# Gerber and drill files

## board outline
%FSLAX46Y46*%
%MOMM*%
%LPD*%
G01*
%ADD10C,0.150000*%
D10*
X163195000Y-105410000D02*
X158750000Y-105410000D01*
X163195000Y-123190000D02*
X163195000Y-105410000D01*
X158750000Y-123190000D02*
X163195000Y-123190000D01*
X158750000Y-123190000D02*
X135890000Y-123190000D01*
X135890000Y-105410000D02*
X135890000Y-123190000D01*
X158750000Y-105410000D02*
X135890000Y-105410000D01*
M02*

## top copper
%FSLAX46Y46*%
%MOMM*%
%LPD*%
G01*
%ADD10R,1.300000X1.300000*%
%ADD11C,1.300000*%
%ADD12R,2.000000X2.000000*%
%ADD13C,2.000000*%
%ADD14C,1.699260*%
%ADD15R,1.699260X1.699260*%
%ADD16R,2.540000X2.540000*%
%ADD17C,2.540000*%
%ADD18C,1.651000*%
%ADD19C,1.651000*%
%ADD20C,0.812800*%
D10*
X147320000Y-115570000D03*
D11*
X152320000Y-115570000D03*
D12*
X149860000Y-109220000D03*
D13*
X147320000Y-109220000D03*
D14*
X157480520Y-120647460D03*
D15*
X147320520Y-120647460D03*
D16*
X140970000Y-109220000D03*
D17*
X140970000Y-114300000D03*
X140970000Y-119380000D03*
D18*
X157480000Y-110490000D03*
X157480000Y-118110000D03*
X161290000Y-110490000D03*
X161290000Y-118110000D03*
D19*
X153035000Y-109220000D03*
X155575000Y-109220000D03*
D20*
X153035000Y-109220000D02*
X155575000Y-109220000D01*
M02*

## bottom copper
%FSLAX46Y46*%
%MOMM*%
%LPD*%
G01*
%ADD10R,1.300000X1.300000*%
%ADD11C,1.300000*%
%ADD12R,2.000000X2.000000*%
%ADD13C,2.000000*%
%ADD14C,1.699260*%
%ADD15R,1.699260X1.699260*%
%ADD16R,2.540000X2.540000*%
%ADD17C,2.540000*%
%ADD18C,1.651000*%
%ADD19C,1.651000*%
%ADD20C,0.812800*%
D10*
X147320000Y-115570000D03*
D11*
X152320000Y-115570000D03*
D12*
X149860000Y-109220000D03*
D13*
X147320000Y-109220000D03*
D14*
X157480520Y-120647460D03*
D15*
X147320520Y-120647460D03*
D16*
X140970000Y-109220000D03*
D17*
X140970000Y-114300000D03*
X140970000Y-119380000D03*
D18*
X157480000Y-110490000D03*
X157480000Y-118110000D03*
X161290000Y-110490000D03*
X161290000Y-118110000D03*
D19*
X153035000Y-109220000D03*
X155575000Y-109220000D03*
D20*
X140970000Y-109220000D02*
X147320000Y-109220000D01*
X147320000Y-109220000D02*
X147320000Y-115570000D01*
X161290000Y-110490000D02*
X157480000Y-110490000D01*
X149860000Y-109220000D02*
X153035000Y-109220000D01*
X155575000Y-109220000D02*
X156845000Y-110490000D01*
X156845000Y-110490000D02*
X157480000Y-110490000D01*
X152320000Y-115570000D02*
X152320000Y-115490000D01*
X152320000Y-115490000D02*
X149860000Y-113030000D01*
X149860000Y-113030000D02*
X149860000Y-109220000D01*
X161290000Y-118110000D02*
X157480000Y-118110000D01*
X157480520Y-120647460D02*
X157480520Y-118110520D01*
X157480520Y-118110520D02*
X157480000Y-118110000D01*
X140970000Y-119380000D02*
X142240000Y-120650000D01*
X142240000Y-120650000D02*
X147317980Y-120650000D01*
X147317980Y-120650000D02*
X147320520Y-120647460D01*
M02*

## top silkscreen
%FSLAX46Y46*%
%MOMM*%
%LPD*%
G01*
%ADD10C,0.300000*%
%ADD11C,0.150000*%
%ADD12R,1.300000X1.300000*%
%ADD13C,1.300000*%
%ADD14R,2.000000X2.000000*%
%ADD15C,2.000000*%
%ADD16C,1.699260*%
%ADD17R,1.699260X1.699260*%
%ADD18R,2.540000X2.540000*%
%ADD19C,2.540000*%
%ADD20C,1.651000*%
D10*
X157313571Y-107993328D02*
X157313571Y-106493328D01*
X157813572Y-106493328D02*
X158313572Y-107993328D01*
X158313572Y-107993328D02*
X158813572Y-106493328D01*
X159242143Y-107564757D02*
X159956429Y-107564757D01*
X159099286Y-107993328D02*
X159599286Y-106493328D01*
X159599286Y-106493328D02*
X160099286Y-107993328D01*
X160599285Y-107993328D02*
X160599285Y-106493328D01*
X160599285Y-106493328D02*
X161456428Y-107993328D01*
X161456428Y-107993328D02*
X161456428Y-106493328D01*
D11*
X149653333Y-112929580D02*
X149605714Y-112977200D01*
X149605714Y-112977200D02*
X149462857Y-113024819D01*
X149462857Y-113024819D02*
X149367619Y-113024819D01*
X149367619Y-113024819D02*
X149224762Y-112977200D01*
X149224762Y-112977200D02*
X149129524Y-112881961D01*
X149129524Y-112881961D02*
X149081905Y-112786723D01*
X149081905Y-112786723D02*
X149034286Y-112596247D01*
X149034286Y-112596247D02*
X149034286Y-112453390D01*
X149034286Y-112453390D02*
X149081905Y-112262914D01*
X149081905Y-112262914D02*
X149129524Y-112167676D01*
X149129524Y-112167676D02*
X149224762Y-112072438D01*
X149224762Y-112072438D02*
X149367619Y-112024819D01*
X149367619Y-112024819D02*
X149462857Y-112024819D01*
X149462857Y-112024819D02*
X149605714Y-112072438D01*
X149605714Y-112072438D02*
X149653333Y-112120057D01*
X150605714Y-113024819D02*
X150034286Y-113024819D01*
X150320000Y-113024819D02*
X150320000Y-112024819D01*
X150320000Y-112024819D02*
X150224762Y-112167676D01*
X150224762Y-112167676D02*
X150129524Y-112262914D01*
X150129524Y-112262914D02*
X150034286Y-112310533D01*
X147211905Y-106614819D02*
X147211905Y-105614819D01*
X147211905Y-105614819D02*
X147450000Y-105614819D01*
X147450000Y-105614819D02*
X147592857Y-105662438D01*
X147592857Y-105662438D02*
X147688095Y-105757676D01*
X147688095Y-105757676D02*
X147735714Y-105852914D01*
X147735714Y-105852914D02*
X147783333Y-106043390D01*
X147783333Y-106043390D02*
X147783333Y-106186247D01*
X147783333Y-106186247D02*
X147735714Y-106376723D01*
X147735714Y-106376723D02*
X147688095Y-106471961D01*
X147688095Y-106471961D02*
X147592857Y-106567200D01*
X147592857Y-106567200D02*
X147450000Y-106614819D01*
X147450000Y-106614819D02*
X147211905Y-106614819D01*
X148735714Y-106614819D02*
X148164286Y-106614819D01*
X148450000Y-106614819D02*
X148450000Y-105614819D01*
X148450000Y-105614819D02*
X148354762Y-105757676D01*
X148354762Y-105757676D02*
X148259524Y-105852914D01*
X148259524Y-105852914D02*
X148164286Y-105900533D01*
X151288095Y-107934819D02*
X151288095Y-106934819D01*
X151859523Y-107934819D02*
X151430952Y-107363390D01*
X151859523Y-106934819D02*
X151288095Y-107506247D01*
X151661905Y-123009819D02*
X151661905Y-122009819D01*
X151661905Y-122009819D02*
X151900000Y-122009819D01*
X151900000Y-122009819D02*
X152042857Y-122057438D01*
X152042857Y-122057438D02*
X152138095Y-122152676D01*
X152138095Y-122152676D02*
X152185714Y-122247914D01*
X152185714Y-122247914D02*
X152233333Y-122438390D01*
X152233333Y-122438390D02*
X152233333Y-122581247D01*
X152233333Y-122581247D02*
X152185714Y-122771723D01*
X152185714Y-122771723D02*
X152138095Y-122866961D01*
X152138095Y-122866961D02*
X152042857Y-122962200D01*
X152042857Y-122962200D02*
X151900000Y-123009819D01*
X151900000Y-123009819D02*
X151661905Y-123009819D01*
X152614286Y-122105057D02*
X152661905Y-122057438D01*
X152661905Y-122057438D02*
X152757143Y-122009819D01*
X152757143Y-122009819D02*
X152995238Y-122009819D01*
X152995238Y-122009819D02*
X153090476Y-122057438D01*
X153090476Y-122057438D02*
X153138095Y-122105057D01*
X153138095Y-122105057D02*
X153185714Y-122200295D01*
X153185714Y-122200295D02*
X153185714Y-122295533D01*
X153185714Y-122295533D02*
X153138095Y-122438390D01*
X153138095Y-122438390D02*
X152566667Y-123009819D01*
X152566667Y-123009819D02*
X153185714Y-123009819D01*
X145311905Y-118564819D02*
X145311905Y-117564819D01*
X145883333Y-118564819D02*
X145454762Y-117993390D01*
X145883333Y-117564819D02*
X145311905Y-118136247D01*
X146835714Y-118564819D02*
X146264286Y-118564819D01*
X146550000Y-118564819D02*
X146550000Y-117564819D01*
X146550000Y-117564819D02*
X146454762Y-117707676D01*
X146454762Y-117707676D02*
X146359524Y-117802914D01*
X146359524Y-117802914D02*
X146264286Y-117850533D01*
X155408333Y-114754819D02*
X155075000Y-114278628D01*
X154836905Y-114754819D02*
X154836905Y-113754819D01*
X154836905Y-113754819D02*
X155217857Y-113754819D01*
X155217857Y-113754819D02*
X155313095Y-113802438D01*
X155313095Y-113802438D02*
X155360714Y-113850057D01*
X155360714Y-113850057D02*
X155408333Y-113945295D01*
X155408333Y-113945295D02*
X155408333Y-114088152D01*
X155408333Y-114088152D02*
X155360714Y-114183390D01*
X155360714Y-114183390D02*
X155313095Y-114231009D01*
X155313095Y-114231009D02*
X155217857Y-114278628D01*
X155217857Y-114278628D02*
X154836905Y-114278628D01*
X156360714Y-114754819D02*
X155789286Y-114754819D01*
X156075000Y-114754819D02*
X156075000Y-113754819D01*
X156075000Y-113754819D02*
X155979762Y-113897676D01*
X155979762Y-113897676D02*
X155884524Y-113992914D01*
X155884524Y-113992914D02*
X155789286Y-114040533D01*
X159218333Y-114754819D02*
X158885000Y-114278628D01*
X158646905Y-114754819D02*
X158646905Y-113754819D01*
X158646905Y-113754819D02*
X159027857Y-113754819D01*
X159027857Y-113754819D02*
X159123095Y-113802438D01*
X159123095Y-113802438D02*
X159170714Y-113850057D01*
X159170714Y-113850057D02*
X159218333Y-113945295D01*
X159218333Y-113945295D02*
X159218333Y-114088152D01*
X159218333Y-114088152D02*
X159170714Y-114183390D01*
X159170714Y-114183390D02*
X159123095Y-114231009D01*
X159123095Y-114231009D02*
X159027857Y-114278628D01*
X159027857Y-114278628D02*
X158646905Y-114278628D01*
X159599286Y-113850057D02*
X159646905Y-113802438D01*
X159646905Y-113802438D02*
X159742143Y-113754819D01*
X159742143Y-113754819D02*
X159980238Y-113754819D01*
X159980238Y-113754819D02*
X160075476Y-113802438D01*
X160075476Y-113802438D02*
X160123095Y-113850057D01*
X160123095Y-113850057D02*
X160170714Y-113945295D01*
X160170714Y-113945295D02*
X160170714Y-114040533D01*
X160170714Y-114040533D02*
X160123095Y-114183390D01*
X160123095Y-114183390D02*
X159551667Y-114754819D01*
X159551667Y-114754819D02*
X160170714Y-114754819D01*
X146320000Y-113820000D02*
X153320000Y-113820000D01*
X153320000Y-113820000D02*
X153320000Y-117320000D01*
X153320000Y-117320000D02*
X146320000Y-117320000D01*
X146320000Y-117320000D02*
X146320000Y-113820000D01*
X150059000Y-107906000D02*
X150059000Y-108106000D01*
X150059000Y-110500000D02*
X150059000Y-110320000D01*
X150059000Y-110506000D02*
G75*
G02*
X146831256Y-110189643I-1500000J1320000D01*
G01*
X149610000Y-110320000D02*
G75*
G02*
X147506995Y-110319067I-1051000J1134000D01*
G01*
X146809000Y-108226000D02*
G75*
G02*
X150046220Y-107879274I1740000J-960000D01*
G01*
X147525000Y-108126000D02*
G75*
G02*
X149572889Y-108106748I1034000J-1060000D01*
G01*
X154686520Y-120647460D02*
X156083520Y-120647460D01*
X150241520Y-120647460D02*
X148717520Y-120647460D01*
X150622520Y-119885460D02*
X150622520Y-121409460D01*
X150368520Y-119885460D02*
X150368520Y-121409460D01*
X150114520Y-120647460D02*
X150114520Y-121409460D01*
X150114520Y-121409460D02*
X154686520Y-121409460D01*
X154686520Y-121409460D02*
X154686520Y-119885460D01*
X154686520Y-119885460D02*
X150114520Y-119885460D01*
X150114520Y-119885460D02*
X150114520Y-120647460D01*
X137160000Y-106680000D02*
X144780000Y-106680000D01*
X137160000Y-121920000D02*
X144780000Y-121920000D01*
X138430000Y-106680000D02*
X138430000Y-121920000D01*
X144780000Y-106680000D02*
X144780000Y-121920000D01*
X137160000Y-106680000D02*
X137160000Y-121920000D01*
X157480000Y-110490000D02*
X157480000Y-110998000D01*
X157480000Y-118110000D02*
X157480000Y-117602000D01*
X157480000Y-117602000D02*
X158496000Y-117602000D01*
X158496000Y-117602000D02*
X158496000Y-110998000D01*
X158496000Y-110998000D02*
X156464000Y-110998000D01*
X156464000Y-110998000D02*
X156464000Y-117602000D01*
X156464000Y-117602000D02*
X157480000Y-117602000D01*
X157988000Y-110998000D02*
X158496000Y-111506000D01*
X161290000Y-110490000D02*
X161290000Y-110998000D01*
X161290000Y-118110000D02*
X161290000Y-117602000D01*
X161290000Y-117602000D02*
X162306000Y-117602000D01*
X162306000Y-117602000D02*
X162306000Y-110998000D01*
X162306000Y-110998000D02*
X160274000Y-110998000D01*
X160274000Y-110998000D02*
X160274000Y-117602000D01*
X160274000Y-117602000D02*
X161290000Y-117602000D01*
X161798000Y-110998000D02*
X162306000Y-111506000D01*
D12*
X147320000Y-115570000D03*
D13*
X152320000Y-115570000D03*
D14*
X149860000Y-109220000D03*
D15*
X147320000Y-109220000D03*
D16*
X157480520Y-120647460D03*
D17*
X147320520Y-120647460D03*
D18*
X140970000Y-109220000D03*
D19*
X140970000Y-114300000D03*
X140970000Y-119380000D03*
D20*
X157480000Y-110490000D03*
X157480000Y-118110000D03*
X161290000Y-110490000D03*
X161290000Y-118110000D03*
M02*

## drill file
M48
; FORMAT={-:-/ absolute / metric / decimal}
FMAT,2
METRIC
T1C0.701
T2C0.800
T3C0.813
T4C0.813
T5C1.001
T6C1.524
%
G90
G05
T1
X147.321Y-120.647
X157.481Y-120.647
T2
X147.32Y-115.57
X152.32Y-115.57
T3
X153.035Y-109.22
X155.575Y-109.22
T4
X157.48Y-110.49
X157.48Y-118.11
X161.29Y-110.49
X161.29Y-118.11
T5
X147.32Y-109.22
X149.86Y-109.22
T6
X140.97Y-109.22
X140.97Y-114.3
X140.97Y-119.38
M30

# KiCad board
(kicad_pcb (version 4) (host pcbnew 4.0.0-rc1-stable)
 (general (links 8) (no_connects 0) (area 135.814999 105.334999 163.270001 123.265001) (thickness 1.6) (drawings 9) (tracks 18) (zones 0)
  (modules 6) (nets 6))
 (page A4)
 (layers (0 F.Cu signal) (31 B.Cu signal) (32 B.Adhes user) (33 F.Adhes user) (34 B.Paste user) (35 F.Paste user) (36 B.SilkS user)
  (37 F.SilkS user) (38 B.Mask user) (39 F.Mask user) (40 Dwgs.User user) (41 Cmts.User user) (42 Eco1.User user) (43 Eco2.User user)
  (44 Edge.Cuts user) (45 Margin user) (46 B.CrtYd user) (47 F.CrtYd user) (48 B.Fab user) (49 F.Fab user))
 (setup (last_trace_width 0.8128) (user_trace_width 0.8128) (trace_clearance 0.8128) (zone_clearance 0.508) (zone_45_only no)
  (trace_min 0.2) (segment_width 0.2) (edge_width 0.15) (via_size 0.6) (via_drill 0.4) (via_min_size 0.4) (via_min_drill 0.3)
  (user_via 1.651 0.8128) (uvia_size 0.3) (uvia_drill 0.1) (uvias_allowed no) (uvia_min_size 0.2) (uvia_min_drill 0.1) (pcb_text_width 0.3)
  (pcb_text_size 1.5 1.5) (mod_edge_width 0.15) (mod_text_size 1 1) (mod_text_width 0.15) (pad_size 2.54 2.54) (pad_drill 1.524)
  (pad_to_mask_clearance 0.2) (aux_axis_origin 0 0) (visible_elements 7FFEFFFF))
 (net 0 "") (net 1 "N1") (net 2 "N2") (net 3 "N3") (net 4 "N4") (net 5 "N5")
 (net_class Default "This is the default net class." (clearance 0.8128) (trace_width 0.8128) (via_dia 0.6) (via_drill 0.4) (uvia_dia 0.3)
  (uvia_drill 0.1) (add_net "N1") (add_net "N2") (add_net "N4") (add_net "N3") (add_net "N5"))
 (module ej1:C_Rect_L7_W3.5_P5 (layer F.Cu) (at 147.32 115.57)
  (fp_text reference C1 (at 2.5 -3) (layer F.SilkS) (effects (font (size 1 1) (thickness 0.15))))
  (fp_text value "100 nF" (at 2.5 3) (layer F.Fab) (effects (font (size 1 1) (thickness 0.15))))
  (fp_line (start -1 -1.75) (end 6 -1.75) (layer F.SilkS) (width 0.15))
  (fp_line (start 6 -1.75) (end 6 1.75) (layer F.SilkS) (width 0.15))
  (fp_line (start 6 1.75) (end -1 1.75) (layer F.SilkS) (width 0.15))
  (fp_line (start -1 1.75) (end -1 -1.75) (layer F.SilkS) (width 0.15))
  (pad 1 thru_hole rect (at 0 0) (size 1.3 1.3) (drill 0.8) (layers *.Cu *.Mask F.SilkS) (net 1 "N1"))
  (pad 2 thru_hole circle (at 5 0) (size 1.3 1.3) (drill 0.8) (layers *.Cu *.Mask F.SilkS) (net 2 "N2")))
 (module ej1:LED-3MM (layer F.Cu) (at 149.86 109.22 180)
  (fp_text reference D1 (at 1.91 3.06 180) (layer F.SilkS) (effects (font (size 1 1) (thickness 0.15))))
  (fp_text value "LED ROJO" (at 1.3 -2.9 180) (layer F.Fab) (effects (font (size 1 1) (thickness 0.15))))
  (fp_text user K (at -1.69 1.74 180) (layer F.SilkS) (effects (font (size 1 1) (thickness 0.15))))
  (fp_line (start -0.199 1.314) (end -0.199 1.114) (layer F.SilkS) (width 0.15))
  (fp_line (start -0.199 -1.28) (end -0.199 -1.1) (layer F.SilkS) (width 0.15))
  (fp_arc (start 1.301 0.034) (end -0.199 -1.286) (angle 108.5) (layer F.SilkS) (width 0.15))
  (fp_arc (start 1.301 0.034) (end 0.25 -1.1) (angle 85.7) (layer F.SilkS) (width 0.15))
  (fp_arc (start 1.311 0.034) (end 3.051 0.994) (angle 110) (layer F.SilkS) (width 0.15))
  (fp_arc (start 1.301 0.034) (end 2.335 1.094) (angle 87.5) (layer F.SilkS) (width 0.15))
  (pad 1 thru_hole rect (at 0 0 270) (size 2 2) (drill 1.00076) (layers *.Cu *.Mask F.SilkS) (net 2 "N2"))
  (pad 2 thru_hole circle (at 2.54 0 180) (size 2 2) (drill 1.00076) (layers *.Cu *.Mask F.SilkS) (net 1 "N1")))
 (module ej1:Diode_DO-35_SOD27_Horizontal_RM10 (layer F.Cu) (at 147.32 120.65)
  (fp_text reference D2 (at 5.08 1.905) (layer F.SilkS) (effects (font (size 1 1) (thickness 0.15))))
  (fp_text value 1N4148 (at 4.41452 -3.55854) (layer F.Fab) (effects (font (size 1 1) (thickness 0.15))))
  (fp_line (start 7.36652 -0.00254) (end 8.76352 -0.00254) (layer F.SilkS) (width 0.15))
  (fp_line (start 2.92152 -0.00254) (end 1.39752 -0.00254) (layer F.SilkS) (width 0.15))
  (fp_line (start 3.30252 -0.76454) (end 3.30252 0.75946) (layer F.SilkS) (width 0.15))
  (fp_line (start 3.04852 -0.76454) (end 3.04852 0.75946) (layer F.SilkS) (width 0.15))
  (fp_line (start 2.79452 -0.00254) (end 2.79452 0.75946) (layer F.SilkS) (width 0.15))
  (fp_line (start 2.79452 0.75946) (end 7.36652 0.75946) (layer F.SilkS) (width 0.15))
  (fp_line (start 7.36652 0.75946) (end 7.36652 -0.76454) (layer F.SilkS) (width 0.15))
  (fp_line (start 7.36652 -0.76454) (end 2.79452 -0.76454) (layer F.SilkS) (width 0.15))
  (fp_line (start 2.79452 -0.76454) (end 2.79452 -0.00254) (layer F.SilkS) (width 0.15))
  (pad 2 thru_hole circle (at 10.16052 -0.00254 180) (size 1.69926 1.69926) (drill 0.70104) (layers *.Cu *.Mask F.SilkS) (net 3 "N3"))
  (pad 1 thru_hole rect (at 0.00052 -0.00254 180) (size 1.69926 1.69926) (drill 0.70104) (layers *.Cu *.Mask F.SilkS) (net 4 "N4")))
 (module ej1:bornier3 (layer F.Cu) (at 140.97 114.3 270)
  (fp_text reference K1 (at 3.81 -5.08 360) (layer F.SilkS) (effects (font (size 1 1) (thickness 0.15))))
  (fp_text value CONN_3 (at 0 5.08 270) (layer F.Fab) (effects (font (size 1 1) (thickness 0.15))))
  (fp_line (start -7.62 3.81) (end -7.62 -3.81) (layer F.SilkS) (width 0.15))
  (fp_line (start 7.62 3.81) (end 7.62 -3.81) (layer F.SilkS) (width 0.15))
  (fp_line (start -7.62 2.54) (end 7.62 2.54) (layer F.SilkS) (width 0.15))
  (fp_line (start -7.62 -3.81) (end 7.62 -3.81) (layer F.SilkS) (width 0.15))
  (fp_line (start -7.62 3.81) (end 7.62 3.81) (layer F.SilkS) (width 0.15))
  (pad 1 thru_hole rect (at -5.08 0 270) (size 2.54 2.54) (drill 1.524) (layers *.Cu *.Mask F.SilkS) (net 1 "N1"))
  (pad 2 thru_hole circle (at 0 0 270) (size 2.54 2.54) (drill 1.524) (layers *.Cu *.Mask F.SilkS) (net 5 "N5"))
  (pad 3 thru_hole circle (at 5.08 0 270) (size 2.54 2.54) (drill 1.524) (layers *.Cu *.Mask F.SilkS) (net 4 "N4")))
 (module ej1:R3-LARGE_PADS (layer F.Cu) (at 157.48 114.3 270)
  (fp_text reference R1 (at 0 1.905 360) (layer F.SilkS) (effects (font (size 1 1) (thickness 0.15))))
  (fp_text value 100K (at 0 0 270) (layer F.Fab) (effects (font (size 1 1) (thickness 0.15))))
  (fp_line (start -3.81 0) (end -3.302 0) (layer F.SilkS) (width 0.15))
  (fp_line (start 3.81 0) (end 3.302 0) (layer F.SilkS) (width 0.15))
  (fp_line (start 3.302 0) (end 3.302 -1.016) (layer F.SilkS) (width 0.15))
  (fp_line (start 3.302 -1.016) (end -3.302 -1.016) (layer F.SilkS) (width 0.15))
  (fp_line (start -3.302 -1.016) (end -3.302 1.016) (layer F.SilkS) (width 0.15))
  (fp_line (start -3.302 1.016) (end 3.302 1.016) (layer F.SilkS) (width 0.15))
  (fp_line (start 3.302 1.016) (end 3.302 0) (layer F.SilkS) (width 0.15))
  (fp_line (start -3.302 -0.508) (end -2.794 -1.016) (layer F.SilkS) (width 0.15))
  (pad 1 thru_hole circle (at -3.81 0 270) (size 1.651 1.651) (drill 0.8128) (layers *.Cu *.Mask F.SilkS) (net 2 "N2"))
  (pad 2 thru_hole circle (at 3.81 0 270) (size 1.651 1.651) (drill 0.8128) (layers *.Cu *.Mask F.SilkS) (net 3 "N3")))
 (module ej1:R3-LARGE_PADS (layer F.Cu) (at 161.29 114.3 270)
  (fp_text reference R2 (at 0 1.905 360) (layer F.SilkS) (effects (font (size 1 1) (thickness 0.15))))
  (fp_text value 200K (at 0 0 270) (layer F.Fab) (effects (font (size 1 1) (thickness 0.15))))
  (fp_line (start -3.81 0) (end -3.302 0) (layer F.SilkS) (width 0.15))
  (fp_line (start 3.81 0) (end 3.302 0) (layer F.SilkS) (width 0.15))
  (fp_line (start 3.302 0) (end 3.302 -1.016) (layer F.SilkS) (width 0.15))
  (fp_line (start 3.302 -1.016) (end -3.302 -1.016) (layer F.SilkS) (width 0.15))
  (fp_line (start -3.302 -1.016) (end -3.302 1.016) (layer F.SilkS) (width 0.15))
  (fp_line (start -3.302 1.016) (end 3.302 1.016) (layer F.SilkS) (width 0.15))
  (fp_line (start 3.302 1.016) (end 3.302 0) (layer F.SilkS) (width 0.15))
  (fp_line (start -3.302 -0.508) (end -2.794 -1.016) (layer F.SilkS) (width 0.15))
  (pad 1 thru_hole circle (at -3.81 0 270) (size 1.651 1.651) (drill 0.8128) (layers *.Cu *.Mask F.SilkS) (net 2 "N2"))
  (pad 2 thru_hole circle (at 3.81 0 270) (size 1.651 1.651) (drill 0.8128) (layers *.Cu *.Mask F.SilkS) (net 3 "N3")))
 (gr_line (start 163.195 105.41) (end 158.75 105.41) (angle 90) (layer Edge.Cuts) (width 0.15))
 (gr_line (start 163.195 123.19) (end 163.195 105.41) (angle 90) (layer Edge.Cuts) (width 0.15))
 (gr_line (start 158.75 123.19) (end 163.195 123.19) (angle 90) (layer Edge.Cuts) (width 0.15))
 (gr_line (start 158.75 123.19) (end 135.89 123.19) (angle 90) (layer Edge.Cuts) (width 0.15))
 (gr_line (start 135.89 105.41) (end 135.89 123.19) (angle 90) (layer Edge.Cuts) (width 0.15))
 (gr_line (start 158.75 105.41) (end 135.89 105.41) (angle 90) (layer Edge.Cuts) (width 0.15))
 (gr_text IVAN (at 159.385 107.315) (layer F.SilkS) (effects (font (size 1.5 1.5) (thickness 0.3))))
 (segment (start 140.97 109.22) (end 147.32 109.22) (width 0.8128) (layer B.Cu) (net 1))
 (segment (start 147.32 109.22) (end 147.32 115.57) (width 0.8128) (layer B.Cu) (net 1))
 (segment (start 161.29 110.49) (end 157.48 110.49) (width 0.8128) (layer B.Cu) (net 2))
 (segment (start 149.86 109.22) (end 153.035 109.22) (width 0.8128) (layer B.Cu) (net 2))
 (segment (start 153.035 109.22) (end 155.575 109.22) (width 0.8128) (layer F.Cu) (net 2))
 (segment (start 155.575 109.22) (end 156.845 110.49) (width 0.8128) (layer B.Cu) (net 2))
 (segment (start 156.845 110.49) (end 157.48 110.49) (width 0.8128) (layer B.Cu) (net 2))
 (segment (start 152.32 115.57) (end 152.32 115.49) (width 0.8128) (layer B.Cu) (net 2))
 (segment (start 152.32 115.49) (end 149.86 113.03) (width 0.8128) (layer B.Cu) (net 2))
 (segment (start 149.86 113.03) (end 149.86 109.22) (width 0.8128) (layer B.Cu) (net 2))
 (segment (start 161.29 118.11) (end 157.48 118.11) (width 0.8128) (layer B.Cu) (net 3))
 (segment (start 157.48052 120.64746) (end 157.48052 118.11052) (width 0.8128) (layer B.Cu) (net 3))
 (segment (start 157.48052 118.11052) (end 157.48 118.11) (width 0.8128) (layer B.Cu) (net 3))
 (segment (start 140.97 119.38) (end 142.24 120.65) (width 0.8128) (layer B.Cu) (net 4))
 (segment (start 142.24 120.65) (end 147.31798 120.65) (width 0.8128) (layer B.Cu) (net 4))
 (segment (start 147.31798 120.65) (end 147.32052 120.64746) (width 0.8128) (layer B.Cu) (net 4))
 (via (at 153.035 109.22) (size 1.651) (drill 0.8128) (layers F.Cu B.Cu) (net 2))
 (via (at 155.575 109.22) (size 1.651) (drill 0.8128) (layers F.Cu B.Cu) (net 2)))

